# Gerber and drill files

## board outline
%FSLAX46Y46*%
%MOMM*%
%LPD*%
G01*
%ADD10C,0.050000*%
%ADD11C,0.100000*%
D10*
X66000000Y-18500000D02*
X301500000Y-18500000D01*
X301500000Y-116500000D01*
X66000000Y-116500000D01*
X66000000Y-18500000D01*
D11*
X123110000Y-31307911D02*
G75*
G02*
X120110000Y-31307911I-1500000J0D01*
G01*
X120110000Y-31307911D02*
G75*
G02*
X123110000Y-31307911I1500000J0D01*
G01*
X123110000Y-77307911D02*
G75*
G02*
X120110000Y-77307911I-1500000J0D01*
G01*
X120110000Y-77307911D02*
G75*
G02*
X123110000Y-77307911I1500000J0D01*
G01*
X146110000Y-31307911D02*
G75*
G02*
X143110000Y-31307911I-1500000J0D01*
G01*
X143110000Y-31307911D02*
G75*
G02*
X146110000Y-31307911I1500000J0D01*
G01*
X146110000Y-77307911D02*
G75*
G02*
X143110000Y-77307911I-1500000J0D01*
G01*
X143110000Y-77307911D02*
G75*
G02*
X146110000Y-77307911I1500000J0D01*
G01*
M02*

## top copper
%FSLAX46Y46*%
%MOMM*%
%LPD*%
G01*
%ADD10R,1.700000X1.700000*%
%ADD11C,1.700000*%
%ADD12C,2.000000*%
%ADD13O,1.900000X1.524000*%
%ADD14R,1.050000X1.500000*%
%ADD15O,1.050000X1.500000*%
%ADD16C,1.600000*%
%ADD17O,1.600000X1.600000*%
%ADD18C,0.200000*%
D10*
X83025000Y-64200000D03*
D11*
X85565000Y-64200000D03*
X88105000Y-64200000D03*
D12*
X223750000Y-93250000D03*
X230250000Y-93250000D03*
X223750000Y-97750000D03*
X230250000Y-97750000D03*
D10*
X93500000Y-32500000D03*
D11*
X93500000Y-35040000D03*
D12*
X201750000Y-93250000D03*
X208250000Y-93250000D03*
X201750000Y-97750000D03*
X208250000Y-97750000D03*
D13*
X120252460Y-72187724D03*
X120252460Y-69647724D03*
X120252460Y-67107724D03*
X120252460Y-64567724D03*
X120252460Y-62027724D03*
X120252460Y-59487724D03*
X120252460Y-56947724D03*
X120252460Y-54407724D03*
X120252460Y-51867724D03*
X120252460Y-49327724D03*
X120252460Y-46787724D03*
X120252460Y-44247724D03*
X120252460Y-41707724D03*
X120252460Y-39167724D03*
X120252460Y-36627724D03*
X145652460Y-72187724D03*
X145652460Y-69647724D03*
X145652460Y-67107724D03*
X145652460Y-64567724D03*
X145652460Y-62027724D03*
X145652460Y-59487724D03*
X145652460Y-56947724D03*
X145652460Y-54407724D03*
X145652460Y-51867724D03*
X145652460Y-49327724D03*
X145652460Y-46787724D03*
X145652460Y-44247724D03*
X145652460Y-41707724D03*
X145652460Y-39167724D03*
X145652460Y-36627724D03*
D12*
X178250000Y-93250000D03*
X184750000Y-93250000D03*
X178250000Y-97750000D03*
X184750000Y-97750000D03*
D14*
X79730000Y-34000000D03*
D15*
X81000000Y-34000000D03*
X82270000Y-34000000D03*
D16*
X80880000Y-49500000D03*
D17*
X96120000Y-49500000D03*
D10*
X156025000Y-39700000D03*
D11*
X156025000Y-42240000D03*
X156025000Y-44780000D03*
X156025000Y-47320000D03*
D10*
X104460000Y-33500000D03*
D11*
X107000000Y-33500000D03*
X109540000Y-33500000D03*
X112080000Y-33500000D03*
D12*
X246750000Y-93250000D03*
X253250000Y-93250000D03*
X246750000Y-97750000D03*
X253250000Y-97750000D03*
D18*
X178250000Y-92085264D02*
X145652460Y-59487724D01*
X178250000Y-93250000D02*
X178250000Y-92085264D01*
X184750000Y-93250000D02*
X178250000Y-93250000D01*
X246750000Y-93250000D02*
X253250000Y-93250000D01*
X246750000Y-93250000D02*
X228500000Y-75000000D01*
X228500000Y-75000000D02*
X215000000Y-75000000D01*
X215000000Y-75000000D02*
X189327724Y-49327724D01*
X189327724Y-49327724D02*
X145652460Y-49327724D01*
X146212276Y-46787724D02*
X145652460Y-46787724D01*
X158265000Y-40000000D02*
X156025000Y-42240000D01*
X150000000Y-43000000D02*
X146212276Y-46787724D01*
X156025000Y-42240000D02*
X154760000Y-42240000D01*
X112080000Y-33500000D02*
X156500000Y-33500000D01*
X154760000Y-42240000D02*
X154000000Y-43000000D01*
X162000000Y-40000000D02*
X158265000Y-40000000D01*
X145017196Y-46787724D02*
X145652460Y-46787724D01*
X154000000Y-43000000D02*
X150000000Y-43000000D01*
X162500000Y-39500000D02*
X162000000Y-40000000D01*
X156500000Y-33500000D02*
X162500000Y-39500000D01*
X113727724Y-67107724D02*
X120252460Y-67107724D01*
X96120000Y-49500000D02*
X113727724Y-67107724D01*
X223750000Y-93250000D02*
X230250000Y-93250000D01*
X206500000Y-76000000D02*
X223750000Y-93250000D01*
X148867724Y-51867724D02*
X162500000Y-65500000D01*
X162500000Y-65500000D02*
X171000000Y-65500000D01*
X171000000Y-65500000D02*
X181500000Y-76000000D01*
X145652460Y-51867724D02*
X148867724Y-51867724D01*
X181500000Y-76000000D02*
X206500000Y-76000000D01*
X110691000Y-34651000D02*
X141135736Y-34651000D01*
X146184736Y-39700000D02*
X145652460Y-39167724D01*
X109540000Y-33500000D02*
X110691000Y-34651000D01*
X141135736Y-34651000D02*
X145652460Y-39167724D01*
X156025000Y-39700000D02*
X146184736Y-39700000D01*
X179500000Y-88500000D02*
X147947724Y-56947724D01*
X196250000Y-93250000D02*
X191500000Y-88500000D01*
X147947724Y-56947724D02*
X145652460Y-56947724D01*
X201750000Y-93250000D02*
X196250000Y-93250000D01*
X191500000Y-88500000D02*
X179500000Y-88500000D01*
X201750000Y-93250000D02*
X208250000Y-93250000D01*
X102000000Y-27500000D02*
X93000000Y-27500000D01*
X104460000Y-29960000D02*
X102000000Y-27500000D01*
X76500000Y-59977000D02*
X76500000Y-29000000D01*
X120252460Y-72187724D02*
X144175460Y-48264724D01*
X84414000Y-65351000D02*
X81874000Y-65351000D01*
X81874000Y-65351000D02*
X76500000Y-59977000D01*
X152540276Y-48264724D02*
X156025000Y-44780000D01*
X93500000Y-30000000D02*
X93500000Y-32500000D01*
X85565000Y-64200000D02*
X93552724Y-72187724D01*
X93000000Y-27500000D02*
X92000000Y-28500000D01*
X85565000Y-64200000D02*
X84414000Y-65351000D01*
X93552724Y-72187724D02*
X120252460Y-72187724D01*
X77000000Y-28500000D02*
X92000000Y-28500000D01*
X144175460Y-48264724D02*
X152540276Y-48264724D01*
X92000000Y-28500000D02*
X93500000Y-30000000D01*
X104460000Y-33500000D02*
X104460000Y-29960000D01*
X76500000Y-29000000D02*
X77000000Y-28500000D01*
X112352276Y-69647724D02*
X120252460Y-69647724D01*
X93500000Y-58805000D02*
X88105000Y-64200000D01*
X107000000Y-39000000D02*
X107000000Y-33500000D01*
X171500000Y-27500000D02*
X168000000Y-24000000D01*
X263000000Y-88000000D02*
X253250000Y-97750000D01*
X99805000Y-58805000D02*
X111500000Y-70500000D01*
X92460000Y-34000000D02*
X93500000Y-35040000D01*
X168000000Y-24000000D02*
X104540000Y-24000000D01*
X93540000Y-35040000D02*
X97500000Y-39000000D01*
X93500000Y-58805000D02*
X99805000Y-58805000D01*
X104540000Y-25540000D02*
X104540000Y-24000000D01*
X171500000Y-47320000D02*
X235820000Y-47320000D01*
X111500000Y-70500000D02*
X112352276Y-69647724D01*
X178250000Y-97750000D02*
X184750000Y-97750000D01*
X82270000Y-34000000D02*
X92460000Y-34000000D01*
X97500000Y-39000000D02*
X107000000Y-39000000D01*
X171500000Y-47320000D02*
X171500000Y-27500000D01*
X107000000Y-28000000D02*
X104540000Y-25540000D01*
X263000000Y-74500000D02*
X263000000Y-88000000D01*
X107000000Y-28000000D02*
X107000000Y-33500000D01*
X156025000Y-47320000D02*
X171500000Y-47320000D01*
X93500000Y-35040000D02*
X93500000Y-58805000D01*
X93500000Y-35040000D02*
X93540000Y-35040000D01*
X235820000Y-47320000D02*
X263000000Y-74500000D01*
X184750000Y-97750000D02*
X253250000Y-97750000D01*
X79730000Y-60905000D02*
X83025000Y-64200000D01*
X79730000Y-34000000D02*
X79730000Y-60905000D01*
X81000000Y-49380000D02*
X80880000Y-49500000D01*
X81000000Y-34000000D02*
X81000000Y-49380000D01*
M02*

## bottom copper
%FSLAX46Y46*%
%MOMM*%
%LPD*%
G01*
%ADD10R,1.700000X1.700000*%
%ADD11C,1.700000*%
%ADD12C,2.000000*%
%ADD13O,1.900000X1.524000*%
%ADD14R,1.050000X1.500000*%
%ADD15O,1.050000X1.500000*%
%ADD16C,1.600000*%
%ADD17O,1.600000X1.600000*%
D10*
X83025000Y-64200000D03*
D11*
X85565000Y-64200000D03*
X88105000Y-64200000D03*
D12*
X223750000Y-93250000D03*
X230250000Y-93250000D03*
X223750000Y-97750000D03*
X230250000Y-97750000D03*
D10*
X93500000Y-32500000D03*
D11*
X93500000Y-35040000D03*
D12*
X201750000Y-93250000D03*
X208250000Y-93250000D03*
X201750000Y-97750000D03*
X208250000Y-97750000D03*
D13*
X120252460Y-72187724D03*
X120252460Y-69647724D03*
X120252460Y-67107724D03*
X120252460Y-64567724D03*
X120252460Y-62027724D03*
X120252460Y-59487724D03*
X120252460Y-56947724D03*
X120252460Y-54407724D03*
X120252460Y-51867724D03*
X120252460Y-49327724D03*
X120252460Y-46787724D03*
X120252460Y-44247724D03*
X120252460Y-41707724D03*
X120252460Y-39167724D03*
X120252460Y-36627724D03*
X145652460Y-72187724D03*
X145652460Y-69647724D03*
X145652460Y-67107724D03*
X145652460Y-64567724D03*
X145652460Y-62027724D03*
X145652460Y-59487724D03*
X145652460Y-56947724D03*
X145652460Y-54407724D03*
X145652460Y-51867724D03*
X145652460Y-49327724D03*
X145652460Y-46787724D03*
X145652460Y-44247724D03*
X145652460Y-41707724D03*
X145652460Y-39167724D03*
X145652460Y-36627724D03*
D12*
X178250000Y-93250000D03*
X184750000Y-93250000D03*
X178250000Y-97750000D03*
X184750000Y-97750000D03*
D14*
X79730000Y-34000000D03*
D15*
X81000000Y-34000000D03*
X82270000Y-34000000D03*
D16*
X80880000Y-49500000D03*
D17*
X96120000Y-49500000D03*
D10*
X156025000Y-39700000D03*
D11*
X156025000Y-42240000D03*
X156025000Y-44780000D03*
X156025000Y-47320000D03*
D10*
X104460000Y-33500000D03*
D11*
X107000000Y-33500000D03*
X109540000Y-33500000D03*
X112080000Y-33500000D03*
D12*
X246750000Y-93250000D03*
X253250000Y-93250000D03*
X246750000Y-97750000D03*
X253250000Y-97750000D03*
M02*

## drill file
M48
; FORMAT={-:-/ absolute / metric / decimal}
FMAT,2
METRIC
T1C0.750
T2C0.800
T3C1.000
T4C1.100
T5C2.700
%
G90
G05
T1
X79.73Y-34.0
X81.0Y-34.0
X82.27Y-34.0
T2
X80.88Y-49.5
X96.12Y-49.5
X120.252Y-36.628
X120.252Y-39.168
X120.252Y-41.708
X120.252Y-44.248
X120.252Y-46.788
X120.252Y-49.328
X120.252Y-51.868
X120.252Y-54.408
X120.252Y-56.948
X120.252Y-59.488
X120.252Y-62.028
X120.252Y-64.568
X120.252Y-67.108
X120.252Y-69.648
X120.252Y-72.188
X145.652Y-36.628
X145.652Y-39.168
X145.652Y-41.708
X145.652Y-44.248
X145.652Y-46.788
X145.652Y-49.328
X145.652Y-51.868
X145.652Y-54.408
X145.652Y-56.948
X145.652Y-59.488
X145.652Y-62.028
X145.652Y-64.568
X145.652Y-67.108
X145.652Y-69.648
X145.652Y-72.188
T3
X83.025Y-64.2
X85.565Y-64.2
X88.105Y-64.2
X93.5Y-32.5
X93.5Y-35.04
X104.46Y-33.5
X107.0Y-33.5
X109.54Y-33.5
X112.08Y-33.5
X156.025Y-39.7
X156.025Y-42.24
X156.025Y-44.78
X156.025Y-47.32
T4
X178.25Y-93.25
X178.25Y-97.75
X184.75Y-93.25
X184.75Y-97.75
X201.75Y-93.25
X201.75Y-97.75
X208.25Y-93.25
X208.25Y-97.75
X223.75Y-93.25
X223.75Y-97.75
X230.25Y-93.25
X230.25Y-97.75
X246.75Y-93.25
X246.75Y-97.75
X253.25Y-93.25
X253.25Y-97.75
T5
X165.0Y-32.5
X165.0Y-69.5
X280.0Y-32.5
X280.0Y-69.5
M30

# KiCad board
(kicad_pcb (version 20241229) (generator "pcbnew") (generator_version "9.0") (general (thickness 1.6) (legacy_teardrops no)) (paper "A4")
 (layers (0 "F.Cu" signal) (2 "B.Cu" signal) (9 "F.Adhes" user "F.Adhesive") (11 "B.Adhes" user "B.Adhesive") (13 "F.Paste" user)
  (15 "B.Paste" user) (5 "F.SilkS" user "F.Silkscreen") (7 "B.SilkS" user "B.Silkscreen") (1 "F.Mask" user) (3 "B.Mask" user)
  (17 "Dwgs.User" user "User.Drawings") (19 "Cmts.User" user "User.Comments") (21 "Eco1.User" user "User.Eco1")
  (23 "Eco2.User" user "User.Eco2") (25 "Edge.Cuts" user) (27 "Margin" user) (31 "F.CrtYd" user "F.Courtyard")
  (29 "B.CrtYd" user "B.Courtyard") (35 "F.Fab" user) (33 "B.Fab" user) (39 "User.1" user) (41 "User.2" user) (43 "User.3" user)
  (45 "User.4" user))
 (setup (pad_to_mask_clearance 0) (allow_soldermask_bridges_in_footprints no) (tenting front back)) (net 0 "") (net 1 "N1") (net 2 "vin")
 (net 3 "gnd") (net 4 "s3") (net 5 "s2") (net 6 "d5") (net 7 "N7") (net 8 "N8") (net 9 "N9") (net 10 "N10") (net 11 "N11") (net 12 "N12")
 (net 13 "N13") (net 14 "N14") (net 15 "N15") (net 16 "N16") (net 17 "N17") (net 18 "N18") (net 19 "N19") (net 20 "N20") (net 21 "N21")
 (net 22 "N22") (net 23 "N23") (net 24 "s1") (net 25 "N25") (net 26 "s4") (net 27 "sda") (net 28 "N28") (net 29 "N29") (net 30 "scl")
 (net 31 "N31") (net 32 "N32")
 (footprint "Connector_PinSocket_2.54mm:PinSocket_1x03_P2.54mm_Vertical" (layer "F.Cu") (at 83.025 64.2 90)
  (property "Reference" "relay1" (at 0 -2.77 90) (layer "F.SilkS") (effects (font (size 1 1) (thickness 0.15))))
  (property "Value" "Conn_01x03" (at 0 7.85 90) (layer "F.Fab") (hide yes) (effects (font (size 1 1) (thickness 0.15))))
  (pad "1" thru_hole rect (at 0 0 90) (size 1.7 1.7) (drill 1) (layers "*.Cu" "*.Mask") (remove_unused_layers no) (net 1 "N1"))
  (pad "2" thru_hole circle (at 0 2.54 90) (size 1.7 1.7) (drill 1) (layers "*.Cu" "*.Mask") (remove_unused_layers no) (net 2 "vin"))
  (pad "3" thru_hole circle (at 0 5.08 90) (size 1.7 1.7) (drill 1) (layers "*.Cu" "*.Mask") (remove_unused_layers no) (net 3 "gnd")))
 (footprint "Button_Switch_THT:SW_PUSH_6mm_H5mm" (layer "F.Cu") (at 223.75 93.25)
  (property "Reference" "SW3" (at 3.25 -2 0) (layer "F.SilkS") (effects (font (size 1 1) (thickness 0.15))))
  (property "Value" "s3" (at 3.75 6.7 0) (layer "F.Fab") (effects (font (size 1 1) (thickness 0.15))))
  (pad "1" thru_hole circle (at 0 0 90) (size 2 2) (drill 1.1) (layers "*.Cu" "*.Mask") (remove_unused_layers no) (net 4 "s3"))
  (pad "1" thru_hole circle (at 6.5 0 90) (size 2 2) (drill 1.1) (layers "*.Cu" "*.Mask") (remove_unused_layers no) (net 4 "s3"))
  (pad "2" thru_hole circle (at 0 4.5 90) (size 2 2) (drill 1.1) (layers "*.Cu" "*.Mask") (remove_unused_layers no) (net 3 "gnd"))
  (pad "2" thru_hole circle (at 6.5 4.5 90) (size 2 2) (drill 1.1) (layers "*.Cu" "*.Mask") (remove_unused_layers no) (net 3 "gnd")))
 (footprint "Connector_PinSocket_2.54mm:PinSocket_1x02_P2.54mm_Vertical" (layer "F.Cu") (at 93.5 32.5)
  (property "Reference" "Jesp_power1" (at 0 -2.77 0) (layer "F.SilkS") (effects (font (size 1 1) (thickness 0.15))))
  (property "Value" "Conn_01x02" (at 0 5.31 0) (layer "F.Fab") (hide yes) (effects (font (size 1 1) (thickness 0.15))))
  (pad "1" thru_hole rect (at 0 0) (size 1.7 1.7) (drill 1) (layers "*.Cu" "*.Mask") (remove_unused_layers no) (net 2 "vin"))
  (pad "2" thru_hole circle (at 0 2.54) (size 1.7 1.7) (drill 1) (layers "*.Cu" "*.Mask") (remove_unused_layers no) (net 3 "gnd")))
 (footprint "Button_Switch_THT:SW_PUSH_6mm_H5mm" (layer "F.Cu") (at 201.75 93.25)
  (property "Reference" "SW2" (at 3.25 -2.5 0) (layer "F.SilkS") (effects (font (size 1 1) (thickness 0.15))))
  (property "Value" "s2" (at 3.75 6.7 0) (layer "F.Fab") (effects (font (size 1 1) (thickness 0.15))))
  (pad "1" thru_hole circle (at 0 0 90) (size 2 2) (drill 1.1) (layers "*.Cu" "*.Mask") (remove_unused_layers no) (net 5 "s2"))
  (pad "1" thru_hole circle (at 6.5 0 90) (size 2 2) (drill 1.1) (layers "*.Cu" "*.Mask") (remove_unused_layers no) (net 5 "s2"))
  (pad "2" thru_hole circle (at 0 4.5 90) (size 2 2) (drill 1.1) (layers "*.Cu" "*.Mask") (remove_unused_layers no) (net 3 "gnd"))
  (pad "2" thru_hole circle (at 6.5 4.5 90) (size 2 2) (drill 1.1) (layers "*.Cu" "*.Mask") (remove_unused_layers no) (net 3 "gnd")))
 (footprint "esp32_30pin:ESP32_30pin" (layer "F.Cu") (at 132.18 55.167911)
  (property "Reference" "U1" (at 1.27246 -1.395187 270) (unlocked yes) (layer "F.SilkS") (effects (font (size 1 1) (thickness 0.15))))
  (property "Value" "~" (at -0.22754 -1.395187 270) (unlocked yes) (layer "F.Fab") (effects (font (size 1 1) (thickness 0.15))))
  (fp_circle (center -10.57 -23.86) (end -10.57 -22.36) (stroke (width 0.1) (type default)) (fill no) (layer "Edge.Cuts"))
  (fp_circle (center -10.57 22.14) (end -10.57 23.64) (stroke (width 0.1) (type default)) (fill no) (layer "Edge.Cuts"))
  (fp_circle (center 12.43 -23.86) (end 12.43 -22.36) (stroke (width 0.1) (type default)) (fill no) (layer "Edge.Cuts"))
  (fp_circle (center 12.43 22.14) (end 12.43 23.64) (stroke (width 0.1) (type default)) (fill no) (layer "Edge.Cuts"))
  (pad "1" thru_hole oval (at -11.92754 17.019813 270) (size 1.524 1.9) (drill 0.8) (layers "*.Cu" "*.Mask") (remove_unused_layers no)
   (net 2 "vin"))
  (pad "2" thru_hole oval (at -11.92754 14.479813 270) (size 1.524 1.9) (drill 0.8) (layers "*.Cu" "*.Mask") (remove_unused_layers no)
   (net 3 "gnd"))
  (pad "3" thru_hole oval (at -11.92754 11.939813 270) (size 1.524 1.9) (drill 0.8) (layers "*.Cu" "*.Mask") (remove_unused_layers no)
   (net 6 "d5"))
  (pad "4" thru_hole oval (at -11.92754 9.399813 270) (size 1.524 1.9) (drill 0.8) (layers "*.Cu" "*.Mask") (remove_unused_layers no)
   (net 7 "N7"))
  (pad "5" thru_hole oval (at -11.92754 6.859813 270) (size 1.524 1.9) (drill 0.8) (layers "*.Cu" "*.Mask") (remove_unused_layers no)
   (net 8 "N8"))
  (pad "6" thru_hole oval (at -11.92754 4.319813 270) (size 1.524 1.9) (drill 0.8) (layers "*.Cu" "*.Mask") (remove_unused_layers no)
   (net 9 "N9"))
  (pad "7" thru_hole oval (at -11.92754 1.779813 270) (size 1.524 1.9) (drill 0.8) (layers "*.Cu" "*.Mask") (remove_unused_layers no)
   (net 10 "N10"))
  (pad "8" thru_hole oval (at -11.92754 -0.760187 270) (size 1.524 1.9) (drill 0.8) (layers "*.Cu" "*.Mask") (remove_unused_layers no)
   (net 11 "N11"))
  (pad "9" thru_hole oval (at -11.92754 -3.300187 270) (size 1.524 1.9) (drill 0.8) (layers "*.Cu" "*.Mask") (remove_unused_layers no)
   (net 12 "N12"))
  (pad "10" thru_hole oval (at -11.92754 -5.840187 270) (size 1.524 1.9) (drill 0.8) (layers "*.Cu" "*.Mask") (remove_unused_layers no)
   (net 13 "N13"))
  (pad "11" thru_hole oval (at -11.92754 -8.380187 270) (size 1.524 1.9) (drill 0.8) (layers "*.Cu" "*.Mask") (remove_unused_layers no)
   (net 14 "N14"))
  (pad "12" thru_hole oval (at -11.92754 -10.920187 270) (size 1.524 1.9) (drill 0.8) (layers "*.Cu" "*.Mask") (remove_unused_layers no)
   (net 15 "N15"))
  (pad "13" thru_hole oval (at -11.92754 -13.460187 270) (size 1.524 1.9) (drill 0.8) (layers "*.Cu" "*.Mask") (remove_unused_layers no)
   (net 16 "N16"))
  (pad "14" thru_hole oval (at -11.92754 -16.000187 270) (size 1.524 1.9) (drill 0.8) (layers "*.Cu" "*.Mask") (remove_unused_layers no)
   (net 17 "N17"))
  (pad "15" thru_hole oval (at -11.92754 -18.540187 270) (size 1.524 1.9) (drill 0.8) (layers "*.Cu" "*.Mask") (remove_unused_layers no)
   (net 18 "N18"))
  (pad "16" thru_hole oval (at 13.47246 17.019813 270) (size 1.524 1.9) (drill 0.8) (layers "*.Cu" "*.Mask") (remove_unused_layers no)
   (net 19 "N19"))
  (pad "17" thru_hole oval (at 13.47246 14.479813 270) (size 1.524 1.9) (drill 0.8) (layers "*.Cu" "*.Mask") (remove_unused_layers no)
   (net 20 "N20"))
  (pad "18" thru_hole oval (at 13.47246 11.939813 270) (size 1.524 1.9) (drill 0.8) (layers "*.Cu" "*.Mask") (remove_unused_layers no)
   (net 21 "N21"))
  (pad "19" thru_hole oval (at 13.47246 9.399813 270) (size 1.524 1.9) (drill 0.8) (layers "*.Cu" "*.Mask") (remove_unused_layers no)
   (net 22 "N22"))
  (pad "20" thru_hole oval (at 13.47246 6.859813 270) (size 1.524 1.9) (drill 0.8) (layers "*.Cu" "*.Mask" "Dwgs.User")
   (remove_unused_layers no) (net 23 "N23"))
  (pad "21" thru_hole oval (at 13.47246 4.319813 270) (size 1.524 1.9) (drill 0.8) (layers "*.Cu" "*.Mask") (remove_unused_layers no)
   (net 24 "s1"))
  (pad "22" thru_hole oval (at 13.47246 1.779813 270) (size 1.524 1.9) (drill 0.8) (layers "*.Cu" "*.Mask") (remove_unused_layers no)
   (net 5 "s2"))
  (pad "23" thru_hole oval (at 13.47246 -0.760187 270) (size 1.524 1.9) (drill 0.8) (layers "*.Cu" "*.Mask") (remove_unused_layers no)
   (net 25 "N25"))
  (pad "24" thru_hole oval (at 13.47246 -3.300187 270) (size 1.524 1.9) (drill 0.8) (layers "*.Cu" "*.Mask") (remove_unused_layers no)
   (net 4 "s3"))
  (pad "25" thru_hole oval (at 13.47246 -5.840187 270) (size 1.524 1.9) (drill 0.8) (layers "*.Cu" "*.Mask") (remove_unused_layers no)
   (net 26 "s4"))
  (pad "26" thru_hole oval (at 13.47246 -8.380187 270) (size 1.524 1.9) (drill 0.8) (layers "*.Cu" "*.Mask") (remove_unused_layers no)
   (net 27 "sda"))
  (pad "27" thru_hole oval (at 13.47246 -10.920187 270) (size 1.524 1.9) (drill 0.8) (layers "*.Cu" "*.Mask") (remove_unused_layers no)
   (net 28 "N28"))
  (pad "28" thru_hole oval (at 13.47246 -13.460187 270) (size 1.524 1.9) (drill 0.8) (layers "*.Cu" "*.Mask") (remove_unused_layers no)
   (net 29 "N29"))
  (pad "29" thru_hole oval (at 13.47246 -16.000187 270) (size 1.524 1.9) (drill 0.8) (layers "*.Cu" "*.Mask") (remove_unused_layers no)
   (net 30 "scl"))
  (pad "30" thru_hole oval (at 13.47246 -18.540187 270) (size 1.524 1.9) (drill 0.8) (layers "*.Cu" "*.Mask") (remove_unused_layers no)
   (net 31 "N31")))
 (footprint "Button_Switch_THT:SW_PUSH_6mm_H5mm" (layer "F.Cu") (at 178.25 93.25)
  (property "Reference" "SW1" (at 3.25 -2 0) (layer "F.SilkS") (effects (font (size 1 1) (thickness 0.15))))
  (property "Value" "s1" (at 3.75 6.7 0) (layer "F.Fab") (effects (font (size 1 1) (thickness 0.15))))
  (pad "1" thru_hole circle (at 0 0 90) (size 2 2) (drill 1.1) (layers "*.Cu" "*.Mask") (remove_unused_layers no) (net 24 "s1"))
  (pad "1" thru_hole circle (at 6.5 0 90) (size 2 2) (drill 1.1) (layers "*.Cu" "*.Mask") (remove_unused_layers no) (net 24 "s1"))
  (pad "2" thru_hole circle (at 0 4.5 90) (size 2 2) (drill 1.1) (layers "*.Cu" "*.Mask") (remove_unused_layers no) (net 3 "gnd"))
  (pad "2" thru_hole circle (at 6.5 4.5 90) (size 2 2) (drill 1.1) (layers "*.Cu" "*.Mask") (remove_unused_layers no) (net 3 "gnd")))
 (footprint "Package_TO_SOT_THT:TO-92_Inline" (layer "F.Cu") (at 79.73 34)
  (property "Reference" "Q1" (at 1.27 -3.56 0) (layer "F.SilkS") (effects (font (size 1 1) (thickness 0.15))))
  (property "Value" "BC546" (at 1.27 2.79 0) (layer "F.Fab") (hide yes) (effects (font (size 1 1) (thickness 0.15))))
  (pad "1" thru_hole rect (at 0 0) (size 1.05 1.5) (drill 0.75) (layers "*.Cu" "*.Mask") (remove_unused_layers no) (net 1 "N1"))
  (pad "2" thru_hole oval (at 1.27 0) (size 1.05 1.5) (drill 0.75) (layers "*.Cu" "*.Mask") (remove_unused_layers no) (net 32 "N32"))
  (pad "3" thru_hole oval (at 2.54 0) (size 1.05 1.5) (drill 0.75) (layers "*.Cu" "*.Mask") (remove_unused_layers no) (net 3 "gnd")))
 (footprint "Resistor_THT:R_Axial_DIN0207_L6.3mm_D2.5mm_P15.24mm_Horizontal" (layer "F.Cu") (at 80.88 49.5)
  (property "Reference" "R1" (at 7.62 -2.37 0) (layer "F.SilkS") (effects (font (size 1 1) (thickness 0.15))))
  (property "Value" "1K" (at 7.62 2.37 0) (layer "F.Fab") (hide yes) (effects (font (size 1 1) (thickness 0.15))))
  (pad "1" thru_hole circle (at 0 0) (size 1.6 1.6) (drill 0.8) (layers "*.Cu" "*.Mask") (remove_unused_layers no) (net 32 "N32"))
  (pad "2" thru_hole oval (at 15.24 0) (size 1.6 1.6) (drill 0.8) (layers "*.Cu" "*.Mask") (remove_unused_layers no) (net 6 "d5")))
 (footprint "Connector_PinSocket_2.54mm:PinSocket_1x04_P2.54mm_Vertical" (layer "F.Cu") (at 156.025 39.7)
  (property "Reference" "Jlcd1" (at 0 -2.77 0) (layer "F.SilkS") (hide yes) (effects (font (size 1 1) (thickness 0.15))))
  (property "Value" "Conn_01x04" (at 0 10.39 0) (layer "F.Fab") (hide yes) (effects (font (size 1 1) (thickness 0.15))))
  (pad "1" thru_hole rect (at 0 0) (size 1.7 1.7) (drill 1) (layers "*.Cu" "*.Mask") (remove_unused_layers no) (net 30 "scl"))
  (pad "2" thru_hole circle (at 0 2.54) (size 1.7 1.7) (drill 1) (layers "*.Cu" "*.Mask") (remove_unused_layers no) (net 27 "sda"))
  (pad "3" thru_hole circle (at 0 5.08) (size 1.7 1.7) (drill 1) (layers "*.Cu" "*.Mask") (remove_unused_layers no) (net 2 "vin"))
  (pad "4" thru_hole circle (at 0 7.62) (size 1.7 1.7) (drill 1) (layers "*.Cu" "*.Mask") (remove_unused_layers no) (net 3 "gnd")))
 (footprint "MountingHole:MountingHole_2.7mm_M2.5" (layer "F.Cu") (at 280 32.5)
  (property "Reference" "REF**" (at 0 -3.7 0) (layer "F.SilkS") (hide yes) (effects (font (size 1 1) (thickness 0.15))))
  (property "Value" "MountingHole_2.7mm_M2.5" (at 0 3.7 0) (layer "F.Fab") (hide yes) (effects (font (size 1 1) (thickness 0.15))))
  (pad "" np_thru_hole circle (at 0 0) (size 2.7 2.7) (drill 2.7) (layers "*.Cu" "*.Mask")))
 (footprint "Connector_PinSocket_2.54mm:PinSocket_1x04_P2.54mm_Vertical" (layer "F.Cu") (at 104.46 33.5 90)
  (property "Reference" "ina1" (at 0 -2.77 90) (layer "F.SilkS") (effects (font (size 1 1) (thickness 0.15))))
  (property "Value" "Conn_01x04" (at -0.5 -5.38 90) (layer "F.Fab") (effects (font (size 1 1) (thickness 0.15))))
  (pad "1" thru_hole rect (at 0 0 90) (size 1.7 1.7) (drill 1) (layers "*.Cu" "*.Mask") (remove_unused_layers no) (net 2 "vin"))
  (pad "2" thru_hole circle (at 0 2.54 90) (size 1.7 1.7) (drill 1) (layers "*.Cu" "*.Mask") (remove_unused_layers no) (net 3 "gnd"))
  (pad "3" thru_hole circle (at 0 5.08 90) (size 1.7 1.7) (drill 1) (layers "*.Cu" "*.Mask") (remove_unused_layers no) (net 30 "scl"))
  (pad "4" thru_hole circle (at 0 7.62 90) (size 1.7 1.7) (drill 1) (layers "*.Cu" "*.Mask") (remove_unused_layers no) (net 27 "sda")))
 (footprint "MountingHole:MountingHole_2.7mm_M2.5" (layer "F.Cu") (at 280 69.5)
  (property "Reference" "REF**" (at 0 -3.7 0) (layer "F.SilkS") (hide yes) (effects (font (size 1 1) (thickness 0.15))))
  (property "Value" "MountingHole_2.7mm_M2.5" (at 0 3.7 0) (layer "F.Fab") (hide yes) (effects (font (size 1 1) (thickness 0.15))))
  (pad "" np_thru_hole circle (at 0 0) (size 2.7 2.7) (drill 2.7) (layers "*.Cu" "*.Mask")))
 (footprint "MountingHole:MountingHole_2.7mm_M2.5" (layer "F.Cu") (at 165 32.5)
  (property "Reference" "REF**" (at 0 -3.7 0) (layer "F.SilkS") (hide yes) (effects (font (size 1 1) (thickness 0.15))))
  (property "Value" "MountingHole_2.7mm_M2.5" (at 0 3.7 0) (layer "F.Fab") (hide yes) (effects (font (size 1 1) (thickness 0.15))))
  (pad "" np_thru_hole circle (at 0 0) (size 2.7 2.7) (drill 2.7) (layers "*.Cu" "*.Mask")))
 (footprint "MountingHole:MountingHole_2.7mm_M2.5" (layer "F.Cu") (at 165 69.5)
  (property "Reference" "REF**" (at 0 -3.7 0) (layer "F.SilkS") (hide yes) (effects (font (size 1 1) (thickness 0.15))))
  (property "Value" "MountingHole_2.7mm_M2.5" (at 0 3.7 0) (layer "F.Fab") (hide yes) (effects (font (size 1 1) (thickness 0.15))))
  (pad "" np_thru_hole circle (at 0 0) (size 2.7 2.7) (drill 2.7) (layers "*.Cu" "*.Mask")))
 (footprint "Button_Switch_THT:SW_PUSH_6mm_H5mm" (layer "F.Cu") (at 246.75 93.25)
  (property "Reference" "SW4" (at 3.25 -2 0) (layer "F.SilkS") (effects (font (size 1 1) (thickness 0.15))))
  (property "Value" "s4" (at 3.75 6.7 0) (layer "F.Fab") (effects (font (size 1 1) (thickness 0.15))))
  (pad "1" thru_hole circle (at 0 0 90) (size 2 2) (drill 1.1) (layers "*.Cu" "*.Mask") (remove_unused_layers no) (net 26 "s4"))
  (pad "1" thru_hole circle (at 6.5 0 90) (size 2 2) (drill 1.1) (layers "*.Cu" "*.Mask") (remove_unused_layers no) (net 26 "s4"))
  (pad "2" thru_hole circle (at 0 4.5 90) (size 2 2) (drill 1.1) (layers "*.Cu" "*.Mask") (remove_unused_layers no) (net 3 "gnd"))
  (pad "2" thru_hole circle (at 6.5 4.5 90) (size 2 2) (drill 1.1) (layers "*.Cu" "*.Mask") (remove_unused_layers no) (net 3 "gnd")))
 (gr_rect (start 66 18.5) (end 301.5 116.5) (stroke (width 0.05) (type default)) (fill no) (layer "Edge.Cuts"))
 (segment (start 178.25 92.085264) (end 145.65246 59.487724) (width 0.2) (layer "F.Cu") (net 24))
 (segment (start 178.25 93.25) (end 178.25 92.085264) (width 0.2) (layer "F.Cu") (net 24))
 (segment (start 184.75 93.25) (end 178.25 93.25) (width 0.2) (layer "F.Cu") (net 24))
 (segment (start 246.75 93.25) (end 253.25 93.25) (width 0.2) (layer "F.Cu") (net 26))
 (segment (start 246.75 93.25) (end 228.5 75) (width 0.2) (layer "F.Cu") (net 26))
 (segment (start 228.5 75) (end 215 75) (width 0.2) (layer "F.Cu") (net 26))
 (segment (start 215 75) (end 189.327724 49.327724) (width 0.2) (layer "F.Cu") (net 26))
 (segment (start 189.327724 49.327724) (end 145.65246 49.327724) (width 0.2) (layer "F.Cu") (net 26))
 (segment (start 146.212276 46.787724) (end 145.65246 46.787724) (width 0.2) (layer "F.Cu") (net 27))
 (segment (start 158.265 40) (end 156.025 42.24) (width 0.2) (layer "F.Cu") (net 27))
 (segment (start 150 43) (end 146.212276 46.787724) (width 0.2) (layer "F.Cu") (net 27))
 (segment (start 156.025 42.24) (end 154.76 42.24) (width 0.2) (layer "F.Cu") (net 27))
 (segment (start 112.08 33.5) (end 156.5 33.5) (width 0.2) (layer "F.Cu") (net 27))
 (segment (start 154.76 42.24) (end 154 43) (width 0.2) (layer "F.Cu") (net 27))
 (segment (start 162 40) (end 158.265 40) (width 0.2) (layer "F.Cu") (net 27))
 (segment (start 145.017196 46.787724) (end 145.65246 46.787724) (width 0.2) (layer "F.Cu") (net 27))
 (segment (start 154 43) (end 150 43) (width 0.2) (layer "F.Cu") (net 27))
 (segment (start 162.5 39.5) (end 162 40) (width 0.2) (layer "F.Cu") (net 27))
 (segment (start 156.5 33.5) (end 162.5 39.5) (width 0.2) (layer "F.Cu") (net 27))
 (segment (start 113.727724 67.107724) (end 120.25246 67.107724) (width 0.2) (layer "F.Cu") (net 6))
 (segment (start 96.12 49.5) (end 113.727724 67.107724) (width 0.2) (layer "F.Cu") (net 6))
 (segment (start 223.75 93.25) (end 230.25 93.25) (width 0.2) (layer "F.Cu") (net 4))
 (segment (start 206.5 76) (end 223.75 93.25) (width 0.2) (layer "F.Cu") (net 4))
 (segment (start 148.867724 51.867724) (end 162.5 65.5) (width 0.2) (layer "F.Cu") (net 4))
 (segment (start 162.5 65.5) (end 171 65.5) (width 0.2) (layer "F.Cu") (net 4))
 (segment (start 171 65.5) (end 181.5 76) (width 0.2) (layer "F.Cu") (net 4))
 (segment (start 145.65246 51.867724) (end 148.867724 51.867724) (width 0.2) (layer "F.Cu") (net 4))
 (segment (start 181.5 76) (end 206.5 76) (width 0.2) (layer "F.Cu") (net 4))
 (segment (start 110.691 34.651) (end 141.135736 34.651) (width 0.2) (layer "F.Cu") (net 30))
 (segment (start 146.184736 39.7) (end 145.65246 39.167724) (width 0.2) (layer "F.Cu") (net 30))
 (segment (start 109.54 33.5) (end 110.691 34.651) (width 0.2) (layer "F.Cu") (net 30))
 (segment (start 141.135736 34.651) (end 145.65246 39.167724) (width 0.2) (layer "F.Cu") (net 30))
 (segment (start 156.025 39.7) (end 146.184736 39.7) (width 0.2) (layer "F.Cu") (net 30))
 (segment (start 179.5 88.5) (end 147.947724 56.947724) (width 0.2) (layer "F.Cu") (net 5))
 (segment (start 196.25 93.25) (end 191.5 88.5) (width 0.2) (layer "F.Cu") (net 5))
 (segment (start 147.947724 56.947724) (end 145.65246 56.947724) (width 0.2) (layer "F.Cu") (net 5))
 (segment (start 201.75 93.25) (end 196.25 93.25) (width 0.2) (layer "F.Cu") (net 5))
 (segment (start 191.5 88.5) (end 179.5 88.5) (width 0.2) (layer "F.Cu") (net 5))
 (segment (start 201.75 93.25) (end 208.25 93.25) (width 0.2) (layer "F.Cu") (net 5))
 (segment (start 102 27.5) (end 93 27.5) (width 0.2) (layer "F.Cu") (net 2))
 (segment (start 104.46 29.96) (end 102 27.5) (width 0.2) (layer "F.Cu") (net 2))
 (segment (start 76.5 59.977) (end 76.5 29) (width 0.2) (layer "F.Cu") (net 2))
 (segment (start 120.25246 72.187724) (end 144.17546 48.264724) (width 0.2) (layer "F.Cu") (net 2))
 (segment (start 84.414 65.351) (end 81.874 65.351) (width 0.2) (layer "F.Cu") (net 2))
 (segment (start 81.874 65.351) (end 76.5 59.977) (width 0.2) (layer "F.Cu") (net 2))
 (segment (start 152.540276 48.264724) (end 156.025 44.78) (width 0.2) (layer "F.Cu") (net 2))
 (segment (start 93.5 30) (end 93.5 32.5) (width 0.2) (layer "F.Cu") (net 2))
 (segment (start 85.565 64.2) (end 93.552724 72.187724) (width 0.2) (layer "F.Cu") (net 2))
 (segment (start 93 27.5) (end 92 28.5) (width 0.2) (layer "F.Cu") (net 2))
 (segment (start 85.565 64.2) (end 84.414 65.351) (width 0.2) (layer "F.Cu") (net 2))
 (segment (start 93.552724 72.187724) (end 120.25246 72.187724) (width 0.2) (layer "F.Cu") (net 2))
 (segment (start 77 28.5) (end 92 28.5) (width 0.2) (layer "F.Cu") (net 2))
 (segment (start 144.17546 48.264724) (end 152.540276 48.264724) (width 0.2) (layer "F.Cu") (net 2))
 (segment (start 92 28.5) (end 93.5 30) (width 0.2) (layer "F.Cu") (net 2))
 (segment (start 104.46 33.5) (end 104.46 29.96) (width 0.2) (layer "F.Cu") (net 2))
 (segment (start 76.5 29) (end 77 28.5) (width 0.2) (layer "F.Cu") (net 2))
 (segment (start 112.352276 69.647724) (end 120.25246 69.647724) (width 0.2) (layer "F.Cu") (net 3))
 (segment (start 93.5 58.805) (end 88.105 64.2) (width 0.2) (layer "F.Cu") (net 3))
 (segment (start 107 39) (end 107 33.5) (width 0.2) (layer "F.Cu") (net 3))
 (segment (start 171.5 27.5) (end 168 24) (width 0.2) (layer "F.Cu") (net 3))
 (segment (start 263 88) (end 253.25 97.75) (width 0.2) (layer "F.Cu") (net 3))
 (segment (start 99.805 58.805) (end 111.5 70.5) (width 0.2) (layer "F.Cu") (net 3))
 (segment (start 92.46 34) (end 93.5 35.04) (width 0.2) (layer "F.Cu") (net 3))
 (segment (start 168 24) (end 104.54 24) (width 0.2) (layer "F.Cu") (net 3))
 (segment (start 93.54 35.04) (end 97.5 39) (width 0.2) (layer "F.Cu") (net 3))
 (segment (start 93.5 58.805) (end 99.805 58.805) (width 0.2) (layer "F.Cu") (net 3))
 (segment (start 104.54 25.54) (end 104.54 24) (width 0.2) (layer "F.Cu") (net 3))
 (segment (start 171.5 47.32) (end 235.82 47.32) (width 0.2) (layer "F.Cu") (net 3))
 (segment (start 111.5 70.5) (end 112.352276 69.647724) (width 0.2) (layer "F.Cu") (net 3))
 (segment (start 178.25 97.75) (end 184.75 97.75) (width 0.2) (layer "F.Cu") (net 3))
 (segment (start 82.27 34) (end 92.46 34) (width 0.2) (layer "F.Cu") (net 3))
 (segment (start 97.5 39) (end 107 39) (width 0.2) (layer "F.Cu") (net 3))
 (segment (start 171.5 47.32) (end 171.5 27.5) (width 0.2) (layer "F.Cu") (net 3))
 (segment (start 107 28) (end 104.54 25.54) (width 0.2) (layer "F.Cu") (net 3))
 (segment (start 263 74.5) (end 263 88) (width 0.2) (layer "F.Cu") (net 3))
 (segment (start 107 28) (end 107 33.5) (width 0.2) (layer "F.Cu") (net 3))
 (segment (start 156.025 47.32) (end 171.5 47.32) (width 0.2) (layer "F.Cu") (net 3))
 (segment (start 93.5 35.04) (end 93.5 58.805) (width 0.2) (layer "F.Cu") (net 3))
 (segment (start 93.5 35.04) (end 93.54 35.04) (width 0.2) (layer "F.Cu") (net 3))
 (segment (start 235.82 47.32) (end 263 74.5) (width 0.2) (layer "F.Cu") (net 3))
 (segment (start 184.75 97.75) (end 253.25 97.75) (width 0.2) (layer "F.Cu") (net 3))
 (segment (start 79.73 60.905) (end 83.025 64.2) (width 0.2) (layer "F.Cu") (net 1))
 (segment (start 79.73 34) (end 79.73 60.905) (width 0.2) (layer "F.Cu") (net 1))
 (segment (start 81 49.38) (end 80.88 49.5) (width 0.2) (layer "F.Cu") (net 32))
 (segment (start 81 34) (end 81 49.38) (width 0.2) (layer "F.Cu") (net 32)))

